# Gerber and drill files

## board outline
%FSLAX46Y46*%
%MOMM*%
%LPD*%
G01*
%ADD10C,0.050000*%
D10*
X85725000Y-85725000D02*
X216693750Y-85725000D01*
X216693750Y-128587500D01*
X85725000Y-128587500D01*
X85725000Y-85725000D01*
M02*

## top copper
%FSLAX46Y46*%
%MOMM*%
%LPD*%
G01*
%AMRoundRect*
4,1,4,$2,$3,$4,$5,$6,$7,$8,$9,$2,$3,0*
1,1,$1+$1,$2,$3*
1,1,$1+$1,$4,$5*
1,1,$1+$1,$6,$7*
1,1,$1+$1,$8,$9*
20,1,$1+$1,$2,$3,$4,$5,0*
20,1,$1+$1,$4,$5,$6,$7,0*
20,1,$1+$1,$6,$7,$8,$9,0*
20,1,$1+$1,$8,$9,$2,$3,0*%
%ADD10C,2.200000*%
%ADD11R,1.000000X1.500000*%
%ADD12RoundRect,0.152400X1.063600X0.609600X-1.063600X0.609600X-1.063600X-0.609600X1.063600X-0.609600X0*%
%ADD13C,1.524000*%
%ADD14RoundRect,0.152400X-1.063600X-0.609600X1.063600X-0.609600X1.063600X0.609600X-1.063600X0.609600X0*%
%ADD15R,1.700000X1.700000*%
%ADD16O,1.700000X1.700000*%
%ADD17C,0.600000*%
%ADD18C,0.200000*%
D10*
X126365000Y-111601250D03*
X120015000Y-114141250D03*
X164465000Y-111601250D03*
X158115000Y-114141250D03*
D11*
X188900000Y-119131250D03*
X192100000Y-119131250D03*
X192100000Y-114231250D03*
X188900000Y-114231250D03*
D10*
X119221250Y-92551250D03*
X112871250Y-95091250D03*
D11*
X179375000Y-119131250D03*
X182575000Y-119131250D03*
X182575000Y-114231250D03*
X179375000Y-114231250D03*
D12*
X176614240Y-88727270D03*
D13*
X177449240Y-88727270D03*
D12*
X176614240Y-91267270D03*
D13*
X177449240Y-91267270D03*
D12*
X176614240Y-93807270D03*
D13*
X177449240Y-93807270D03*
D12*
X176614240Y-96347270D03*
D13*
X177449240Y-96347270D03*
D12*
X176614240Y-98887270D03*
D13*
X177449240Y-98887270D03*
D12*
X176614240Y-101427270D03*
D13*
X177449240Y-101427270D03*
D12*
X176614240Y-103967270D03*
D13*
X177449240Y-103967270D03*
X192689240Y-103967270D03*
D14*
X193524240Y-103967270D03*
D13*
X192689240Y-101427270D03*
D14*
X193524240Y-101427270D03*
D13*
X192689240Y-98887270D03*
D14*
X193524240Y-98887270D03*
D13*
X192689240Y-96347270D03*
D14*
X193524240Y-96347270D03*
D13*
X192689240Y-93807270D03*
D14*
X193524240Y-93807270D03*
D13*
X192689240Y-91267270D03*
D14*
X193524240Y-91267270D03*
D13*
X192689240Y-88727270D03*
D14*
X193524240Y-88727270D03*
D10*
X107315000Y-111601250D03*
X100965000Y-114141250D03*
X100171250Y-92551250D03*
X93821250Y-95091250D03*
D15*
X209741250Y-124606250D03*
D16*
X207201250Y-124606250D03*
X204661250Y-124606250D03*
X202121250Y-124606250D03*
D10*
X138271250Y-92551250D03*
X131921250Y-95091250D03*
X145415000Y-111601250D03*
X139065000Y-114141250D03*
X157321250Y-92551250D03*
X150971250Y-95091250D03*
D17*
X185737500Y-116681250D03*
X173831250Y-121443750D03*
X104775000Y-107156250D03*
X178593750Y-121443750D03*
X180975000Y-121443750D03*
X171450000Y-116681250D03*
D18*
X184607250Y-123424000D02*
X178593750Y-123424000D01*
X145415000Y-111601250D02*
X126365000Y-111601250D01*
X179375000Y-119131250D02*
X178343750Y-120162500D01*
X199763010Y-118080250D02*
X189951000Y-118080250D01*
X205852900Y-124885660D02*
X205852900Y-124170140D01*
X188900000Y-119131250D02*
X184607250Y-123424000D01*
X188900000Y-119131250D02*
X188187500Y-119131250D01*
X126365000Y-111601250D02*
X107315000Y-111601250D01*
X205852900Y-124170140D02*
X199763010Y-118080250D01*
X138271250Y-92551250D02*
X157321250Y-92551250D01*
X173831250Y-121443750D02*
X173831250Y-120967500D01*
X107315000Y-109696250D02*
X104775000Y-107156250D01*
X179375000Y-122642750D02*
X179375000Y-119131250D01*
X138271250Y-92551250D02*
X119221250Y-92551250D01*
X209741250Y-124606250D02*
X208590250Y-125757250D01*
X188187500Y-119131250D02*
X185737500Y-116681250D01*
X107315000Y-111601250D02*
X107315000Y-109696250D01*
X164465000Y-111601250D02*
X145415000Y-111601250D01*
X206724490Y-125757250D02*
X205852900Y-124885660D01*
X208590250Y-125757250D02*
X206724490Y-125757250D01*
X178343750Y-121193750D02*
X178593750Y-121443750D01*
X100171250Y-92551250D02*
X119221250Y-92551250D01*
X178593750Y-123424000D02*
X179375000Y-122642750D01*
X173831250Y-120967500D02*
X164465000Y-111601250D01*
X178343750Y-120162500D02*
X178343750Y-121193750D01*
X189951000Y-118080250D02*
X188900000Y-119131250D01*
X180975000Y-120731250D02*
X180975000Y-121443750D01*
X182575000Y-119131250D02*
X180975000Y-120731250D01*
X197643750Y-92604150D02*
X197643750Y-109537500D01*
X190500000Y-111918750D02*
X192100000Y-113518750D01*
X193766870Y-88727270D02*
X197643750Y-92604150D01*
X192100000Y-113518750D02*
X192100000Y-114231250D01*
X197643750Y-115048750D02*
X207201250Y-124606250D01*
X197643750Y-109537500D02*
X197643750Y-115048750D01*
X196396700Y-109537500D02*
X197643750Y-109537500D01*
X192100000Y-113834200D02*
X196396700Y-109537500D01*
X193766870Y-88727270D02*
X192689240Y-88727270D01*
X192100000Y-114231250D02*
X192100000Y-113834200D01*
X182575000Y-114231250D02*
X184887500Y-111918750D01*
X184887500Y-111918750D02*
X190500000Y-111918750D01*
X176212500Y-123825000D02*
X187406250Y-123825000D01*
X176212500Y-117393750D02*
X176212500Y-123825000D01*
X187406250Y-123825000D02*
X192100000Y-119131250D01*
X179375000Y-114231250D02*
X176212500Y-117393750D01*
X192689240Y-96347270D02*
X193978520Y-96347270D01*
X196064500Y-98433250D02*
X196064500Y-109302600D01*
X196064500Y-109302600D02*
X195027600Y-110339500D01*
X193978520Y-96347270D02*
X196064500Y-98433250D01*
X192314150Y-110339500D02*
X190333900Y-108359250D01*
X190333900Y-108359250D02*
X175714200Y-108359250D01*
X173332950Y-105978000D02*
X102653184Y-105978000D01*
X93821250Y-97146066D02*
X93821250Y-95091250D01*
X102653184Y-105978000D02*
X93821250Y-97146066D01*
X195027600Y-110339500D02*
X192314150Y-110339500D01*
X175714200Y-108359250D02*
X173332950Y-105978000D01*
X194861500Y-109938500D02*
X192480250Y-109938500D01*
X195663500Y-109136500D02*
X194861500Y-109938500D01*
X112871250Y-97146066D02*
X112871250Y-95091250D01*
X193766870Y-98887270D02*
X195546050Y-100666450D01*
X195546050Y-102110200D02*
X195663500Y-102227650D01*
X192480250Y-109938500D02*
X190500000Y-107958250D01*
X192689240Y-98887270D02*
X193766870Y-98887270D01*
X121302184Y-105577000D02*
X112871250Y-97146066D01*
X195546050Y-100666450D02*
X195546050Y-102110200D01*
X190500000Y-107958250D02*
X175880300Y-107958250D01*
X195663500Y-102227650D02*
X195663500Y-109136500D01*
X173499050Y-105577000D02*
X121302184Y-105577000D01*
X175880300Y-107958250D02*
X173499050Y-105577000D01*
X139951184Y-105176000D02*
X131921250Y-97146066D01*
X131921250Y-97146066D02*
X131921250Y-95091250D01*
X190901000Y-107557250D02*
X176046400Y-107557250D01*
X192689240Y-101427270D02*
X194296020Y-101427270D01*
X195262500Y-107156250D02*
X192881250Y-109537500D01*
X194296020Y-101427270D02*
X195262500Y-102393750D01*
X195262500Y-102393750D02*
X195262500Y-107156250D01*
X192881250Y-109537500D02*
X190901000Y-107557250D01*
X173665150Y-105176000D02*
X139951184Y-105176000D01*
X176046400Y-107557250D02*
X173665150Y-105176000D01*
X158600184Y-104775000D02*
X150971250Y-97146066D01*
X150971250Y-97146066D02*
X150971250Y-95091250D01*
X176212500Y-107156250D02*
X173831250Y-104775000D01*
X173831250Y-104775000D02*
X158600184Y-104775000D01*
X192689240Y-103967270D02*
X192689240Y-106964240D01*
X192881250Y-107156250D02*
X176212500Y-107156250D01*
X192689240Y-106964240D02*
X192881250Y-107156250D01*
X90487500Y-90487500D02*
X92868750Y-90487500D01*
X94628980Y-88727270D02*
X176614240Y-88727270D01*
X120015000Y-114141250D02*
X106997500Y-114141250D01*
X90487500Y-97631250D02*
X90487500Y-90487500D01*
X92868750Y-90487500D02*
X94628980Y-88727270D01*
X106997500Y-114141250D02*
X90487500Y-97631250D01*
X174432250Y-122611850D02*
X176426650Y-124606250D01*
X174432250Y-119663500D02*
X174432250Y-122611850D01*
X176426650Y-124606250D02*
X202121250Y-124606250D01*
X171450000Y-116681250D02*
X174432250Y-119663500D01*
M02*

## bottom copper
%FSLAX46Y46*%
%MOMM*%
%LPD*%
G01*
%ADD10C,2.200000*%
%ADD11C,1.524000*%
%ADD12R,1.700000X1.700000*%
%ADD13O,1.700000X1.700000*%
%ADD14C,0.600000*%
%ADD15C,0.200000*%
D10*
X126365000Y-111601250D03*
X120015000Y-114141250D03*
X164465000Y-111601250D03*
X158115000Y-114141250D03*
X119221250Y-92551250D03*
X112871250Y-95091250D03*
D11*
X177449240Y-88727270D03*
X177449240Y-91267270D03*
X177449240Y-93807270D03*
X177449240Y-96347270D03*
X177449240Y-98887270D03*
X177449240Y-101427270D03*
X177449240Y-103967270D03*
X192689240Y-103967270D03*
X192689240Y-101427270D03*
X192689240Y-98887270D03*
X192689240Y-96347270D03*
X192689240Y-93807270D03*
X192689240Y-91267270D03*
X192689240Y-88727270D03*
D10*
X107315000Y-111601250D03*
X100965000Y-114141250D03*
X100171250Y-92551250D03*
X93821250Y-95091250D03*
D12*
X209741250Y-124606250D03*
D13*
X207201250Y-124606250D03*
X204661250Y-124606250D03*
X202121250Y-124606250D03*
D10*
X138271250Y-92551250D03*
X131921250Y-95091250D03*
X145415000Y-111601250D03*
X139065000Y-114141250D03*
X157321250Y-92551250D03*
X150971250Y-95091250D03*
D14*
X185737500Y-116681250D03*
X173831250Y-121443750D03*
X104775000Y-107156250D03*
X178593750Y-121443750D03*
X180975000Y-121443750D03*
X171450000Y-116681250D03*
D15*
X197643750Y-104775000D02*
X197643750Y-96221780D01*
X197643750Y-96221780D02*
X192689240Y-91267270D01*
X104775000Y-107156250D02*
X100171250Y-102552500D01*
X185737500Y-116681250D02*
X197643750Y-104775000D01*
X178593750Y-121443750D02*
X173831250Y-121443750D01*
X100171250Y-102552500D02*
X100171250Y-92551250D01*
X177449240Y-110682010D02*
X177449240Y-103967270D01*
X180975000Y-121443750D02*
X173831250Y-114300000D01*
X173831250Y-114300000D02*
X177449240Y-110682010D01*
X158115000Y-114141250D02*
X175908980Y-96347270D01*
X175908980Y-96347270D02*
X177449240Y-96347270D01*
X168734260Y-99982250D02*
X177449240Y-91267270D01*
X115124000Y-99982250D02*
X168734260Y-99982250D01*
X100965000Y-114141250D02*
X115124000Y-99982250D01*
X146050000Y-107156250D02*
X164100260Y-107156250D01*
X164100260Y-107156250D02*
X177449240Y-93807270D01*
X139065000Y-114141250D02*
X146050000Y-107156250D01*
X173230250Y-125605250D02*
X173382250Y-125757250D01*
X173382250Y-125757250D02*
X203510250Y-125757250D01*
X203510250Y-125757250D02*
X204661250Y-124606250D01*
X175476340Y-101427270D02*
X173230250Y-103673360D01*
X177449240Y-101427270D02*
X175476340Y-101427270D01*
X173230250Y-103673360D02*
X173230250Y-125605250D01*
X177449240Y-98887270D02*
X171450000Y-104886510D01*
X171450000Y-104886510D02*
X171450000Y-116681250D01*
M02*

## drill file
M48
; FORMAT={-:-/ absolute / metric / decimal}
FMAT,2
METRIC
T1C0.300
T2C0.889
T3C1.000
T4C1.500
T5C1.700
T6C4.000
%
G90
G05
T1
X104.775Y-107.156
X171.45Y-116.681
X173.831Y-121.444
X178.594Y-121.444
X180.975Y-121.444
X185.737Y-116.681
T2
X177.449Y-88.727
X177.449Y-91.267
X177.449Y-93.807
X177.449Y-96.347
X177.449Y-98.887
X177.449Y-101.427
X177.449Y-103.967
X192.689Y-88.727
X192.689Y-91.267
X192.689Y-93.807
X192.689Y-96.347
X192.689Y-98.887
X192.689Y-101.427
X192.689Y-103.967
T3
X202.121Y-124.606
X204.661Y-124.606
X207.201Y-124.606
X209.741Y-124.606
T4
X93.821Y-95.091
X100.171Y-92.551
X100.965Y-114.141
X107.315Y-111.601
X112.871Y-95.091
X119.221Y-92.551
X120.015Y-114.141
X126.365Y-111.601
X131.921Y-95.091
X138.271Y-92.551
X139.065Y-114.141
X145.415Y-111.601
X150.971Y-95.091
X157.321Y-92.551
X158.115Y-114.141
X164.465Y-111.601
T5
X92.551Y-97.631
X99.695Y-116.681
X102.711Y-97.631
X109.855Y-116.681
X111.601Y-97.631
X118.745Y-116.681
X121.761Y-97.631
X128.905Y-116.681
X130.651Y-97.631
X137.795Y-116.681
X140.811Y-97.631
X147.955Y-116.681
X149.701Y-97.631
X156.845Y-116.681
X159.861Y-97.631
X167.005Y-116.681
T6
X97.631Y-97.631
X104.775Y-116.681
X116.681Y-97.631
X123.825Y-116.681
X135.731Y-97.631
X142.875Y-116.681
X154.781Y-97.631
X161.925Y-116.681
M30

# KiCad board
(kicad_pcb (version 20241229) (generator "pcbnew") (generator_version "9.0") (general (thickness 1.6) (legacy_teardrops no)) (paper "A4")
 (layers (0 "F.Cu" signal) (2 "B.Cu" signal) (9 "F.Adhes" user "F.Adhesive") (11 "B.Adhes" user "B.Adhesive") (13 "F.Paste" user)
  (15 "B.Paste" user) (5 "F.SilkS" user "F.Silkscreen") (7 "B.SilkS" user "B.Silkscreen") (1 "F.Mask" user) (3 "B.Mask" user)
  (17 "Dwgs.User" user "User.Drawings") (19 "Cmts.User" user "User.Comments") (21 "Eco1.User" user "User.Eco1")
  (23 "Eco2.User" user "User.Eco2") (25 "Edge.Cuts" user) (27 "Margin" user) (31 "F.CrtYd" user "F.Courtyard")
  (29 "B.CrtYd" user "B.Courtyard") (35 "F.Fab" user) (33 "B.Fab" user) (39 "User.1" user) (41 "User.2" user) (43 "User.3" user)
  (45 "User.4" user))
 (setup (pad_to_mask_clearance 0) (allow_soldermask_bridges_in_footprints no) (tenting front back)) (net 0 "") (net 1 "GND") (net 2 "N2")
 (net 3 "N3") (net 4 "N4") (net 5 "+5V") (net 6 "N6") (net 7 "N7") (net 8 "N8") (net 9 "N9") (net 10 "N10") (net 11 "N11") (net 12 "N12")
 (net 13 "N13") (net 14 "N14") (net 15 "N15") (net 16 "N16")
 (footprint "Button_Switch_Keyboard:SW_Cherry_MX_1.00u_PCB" (layer "F.Cu") (at 126.365 111.60125)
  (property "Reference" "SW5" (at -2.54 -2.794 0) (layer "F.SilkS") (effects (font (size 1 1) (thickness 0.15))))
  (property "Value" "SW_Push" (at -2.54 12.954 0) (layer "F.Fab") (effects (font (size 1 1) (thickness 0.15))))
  (pad "" np_thru_hole circle (at -7.62 5.08) (size 1.7 1.7) (drill 1.7) (layers "*.Cu" "*.Mask"))
  (pad "" np_thru_hole circle (at -2.54 5.08) (size 4 4) (drill 4) (layers "*.Cu" "*.Mask"))
  (pad "" np_thru_hole circle (at 2.54 5.08) (size 1.7 1.7) (drill 1.7) (layers "*.Cu" "*.Mask"))
  (pad "1" thru_hole circle (at 0 0) (size 2.2 2.2) (drill 1.5) (layers "*.Cu" "*.Mask") (remove_unused_layers no) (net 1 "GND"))
  (pad "2" thru_hole circle (at -6.35 2.54) (size 2.2 2.2) (drill 1.5) (layers "*.Cu" "*.Mask") (remove_unused_layers no) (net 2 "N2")))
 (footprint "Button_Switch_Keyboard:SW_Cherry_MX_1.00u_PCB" (layer "F.Cu") (at 164.465 111.60125)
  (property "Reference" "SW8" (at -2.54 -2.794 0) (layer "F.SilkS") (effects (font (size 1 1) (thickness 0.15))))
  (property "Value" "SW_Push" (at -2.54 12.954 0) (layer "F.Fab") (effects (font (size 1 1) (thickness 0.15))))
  (pad "" np_thru_hole circle (at -7.62 5.08) (size 1.7 1.7) (drill 1.7) (layers "*.Cu" "*.Mask"))
  (pad "" np_thru_hole circle (at -2.54 5.08) (size 4 4) (drill 4) (layers "*.Cu" "*.Mask"))
  (pad "" np_thru_hole circle (at 2.54 5.08) (size 1.7 1.7) (drill 1.7) (layers "*.Cu" "*.Mask"))
  (pad "1" thru_hole circle (at 0 0) (size 2.2 2.2) (drill 1.5) (layers "*.Cu" "*.Mask") (remove_unused_layers no) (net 1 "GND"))
  (pad "2" thru_hole circle (at -6.35 2.54) (size 2.2 2.2) (drill 1.5) (layers "*.Cu" "*.Mask") (remove_unused_layers no) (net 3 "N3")))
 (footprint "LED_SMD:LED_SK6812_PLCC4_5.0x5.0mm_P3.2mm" (layer "F.Cu") (at 190.5 116.68125 90)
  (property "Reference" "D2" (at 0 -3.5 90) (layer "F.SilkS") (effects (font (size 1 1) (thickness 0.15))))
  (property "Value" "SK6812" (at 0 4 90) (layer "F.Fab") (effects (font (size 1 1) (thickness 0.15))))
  (pad "1" smd rect (at -2.45 -1.6 270) (size 1.5 1) (layers "F.Cu" "F.Mask" "F.Paste") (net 1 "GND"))
  (pad "2" smd rect (at -2.45 1.6 270) (size 1.5 1) (layers "F.Cu" "F.Mask" "F.Paste") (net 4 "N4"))
  (pad "3" smd rect (at 2.45 1.6 270) (size 1.5 1) (layers "F.Cu" "F.Mask" "F.Paste") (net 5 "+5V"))
  (pad "4" smd rect (at 2.45 -1.6 270) (size 1.5 1) (layers "F.Cu" "F.Mask" "F.Paste") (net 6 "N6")))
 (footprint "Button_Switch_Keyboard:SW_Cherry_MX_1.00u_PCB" (layer "F.Cu") (at 119.22125 92.55125)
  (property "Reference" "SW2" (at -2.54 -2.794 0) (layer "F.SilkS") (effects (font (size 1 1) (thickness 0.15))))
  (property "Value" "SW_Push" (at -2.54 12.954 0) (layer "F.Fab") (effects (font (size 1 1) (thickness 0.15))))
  (pad "" np_thru_hole circle (at -7.62 5.08) (size 1.7 1.7) (drill 1.7) (layers "*.Cu" "*.Mask"))
  (pad "" np_thru_hole circle (at -2.54 5.08) (size 4 4) (drill 4) (layers "*.Cu" "*.Mask"))
  (pad "" np_thru_hole circle (at 2.54 5.08) (size 1.7 1.7) (drill 1.7) (layers "*.Cu" "*.Mask"))
  (pad "1" thru_hole circle (at 0 0) (size 2.2 2.2) (drill 1.5) (layers "*.Cu" "*.Mask") (remove_unused_layers no) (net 1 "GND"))
  (pad "2" thru_hole circle (at -6.35 2.54) (size 2.2 2.2) (drill 1.5) (layers "*.Cu" "*.Mask") (remove_unused_layers no) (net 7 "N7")))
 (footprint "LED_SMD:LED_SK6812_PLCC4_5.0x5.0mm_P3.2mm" (layer "F.Cu") (at 180.975 116.68125 90)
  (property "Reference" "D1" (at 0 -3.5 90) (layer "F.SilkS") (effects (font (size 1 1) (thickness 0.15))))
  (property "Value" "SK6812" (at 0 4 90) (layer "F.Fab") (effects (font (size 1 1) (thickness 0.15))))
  (pad "1" smd rect (at -2.45 -1.6 270) (size 1.5 1) (layers "F.Cu" "F.Mask" "F.Paste") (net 1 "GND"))
  (pad "2" smd rect (at -2.45 1.6 270) (size 1.5 1) (layers "F.Cu" "F.Mask" "F.Paste") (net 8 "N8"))
  (pad "3" smd rect (at 2.45 1.6 270) (size 1.5 1) (layers "F.Cu" "F.Mask" "F.Paste") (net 5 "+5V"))
  (pad "4" smd rect (at 2.45 -1.6 270) (size 1.5 1) (layers "F.Cu" "F.Mask" "F.Paste") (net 4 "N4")))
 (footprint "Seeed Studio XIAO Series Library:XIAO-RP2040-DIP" (layer "F.Cu") (at 185.06924 96.34727)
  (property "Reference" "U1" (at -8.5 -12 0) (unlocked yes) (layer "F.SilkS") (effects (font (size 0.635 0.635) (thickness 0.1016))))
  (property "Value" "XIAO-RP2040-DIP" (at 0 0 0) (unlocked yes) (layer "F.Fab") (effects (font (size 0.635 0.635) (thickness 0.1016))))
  (pad "1" smd roundrect (at -8.455 -7.62 180) (size 2.432 1.524) (layers "F.Cu" "F.Mask") (roundrect_rratio 0.1) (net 2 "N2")
   (thermal_bridge_angle 45))
  (pad "1" thru_hole circle (at -7.62 -7.62 180) (size 1.524 1.524) (drill 0.889) (layers "*.Cu" "*.Mask") (remove_unused_layers no)
   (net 2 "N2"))
  (pad "2" smd roundrect (at -8.455 -5.08 180) (size 2.432 1.524) (layers "F.Cu" "F.Mask") (roundrect_rratio 0.1) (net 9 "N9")
   (thermal_bridge_angle 45))
  (pad "2" thru_hole circle (at -7.62 -5.08 180) (size 1.524 1.524) (drill 0.889) (layers "*.Cu" "*.Mask") (remove_unused_layers no)
   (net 9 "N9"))
  (pad "3" smd roundrect (at -8.455 -2.54 180) (size 2.432 1.524) (layers "F.Cu" "F.Mask") (roundrect_rratio 0.1) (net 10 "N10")
   (thermal_bridge_angle 45))
  (pad "3" thru_hole circle (at -7.62 -2.54 180) (size 1.524 1.524) (drill 0.889) (layers "*.Cu" "*.Mask") (remove_unused_layers no)
   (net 10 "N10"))
  (pad "4" smd roundrect (at -8.455 0 180) (size 2.432 1.524) (layers "F.Cu" "F.Mask") (roundrect_rratio 0.1) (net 3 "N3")
   (thermal_bridge_angle 45))
  (pad "4" thru_hole circle (at -7.62 0 180) (size 1.524 1.524) (drill 0.889) (layers "*.Cu" "*.Mask") (remove_unused_layers no)
   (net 3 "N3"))
  (pad "5" smd roundrect (at -8.455 2.54 180) (size 2.432 1.524) (layers "F.Cu" "F.Mask") (roundrect_rratio 0.1) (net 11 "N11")
   (thermal_bridge_angle 45))
  (pad "5" thru_hole circle (at -7.62 2.54 180) (size 1.524 1.524) (drill 0.889) (layers "*.Cu" "*.Mask") (remove_unused_layers no)
   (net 11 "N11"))
  (pad "6" smd roundrect (at -8.455 5.08 180) (size 2.432 1.524) (layers "F.Cu" "F.Mask") (roundrect_rratio 0.1) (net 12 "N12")
   (thermal_bridge_angle 45))
  (pad "6" thru_hole circle (at -7.62 5.08 180) (size 1.524 1.524) (drill 0.889) (layers "*.Cu" "*.Mask") (remove_unused_layers no)
   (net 12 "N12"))
  (pad "7" smd roundrect (at -8.455 7.62 180) (size 2.432 1.524) (layers "F.Cu" "F.Mask") (roundrect_rratio 0.1) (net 8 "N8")
   (thermal_bridge_angle 45))
  (pad "7" thru_hole circle (at -7.62 7.62 180) (size 1.524 1.524) (drill 0.889) (layers "*.Cu" "*.Mask") (remove_unused_layers no)
   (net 8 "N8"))
  (pad "8" thru_hole circle (at 7.62 7.62) (size 1.524 1.524) (drill 0.889) (layers "*.Cu" "*.Mask") (remove_unused_layers no)
   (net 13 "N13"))
  (pad "8" smd roundrect (at 8.455 7.62) (size 2.432 1.524) (layers "F.Cu" "F.Mask") (roundrect_rratio 0.1) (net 13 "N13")
   (thermal_bridge_angle 45))
  (pad "9" thru_hole circle (at 7.62 5.08) (size 1.524 1.524) (drill 0.889) (layers "*.Cu" "*.Mask") (remove_unused_layers no)
   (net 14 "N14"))
  (pad "9" smd roundrect (at 8.455 5.08) (size 2.432 1.524) (layers "F.Cu" "F.Mask") (roundrect_rratio 0.1) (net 14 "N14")
   (thermal_bridge_angle 45))
  (pad "10" thru_hole circle (at 7.62 2.54) (size 1.524 1.524) (drill 0.889) (layers "*.Cu" "*.Mask") (remove_unused_layers no) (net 7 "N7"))
  (pad "10" smd roundrect (at 8.455 2.54) (size 2.432 1.524) (layers "F.Cu" "F.Mask") (roundrect_rratio 0.1) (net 7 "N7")
   (thermal_bridge_angle 45))
  (pad "11" thru_hole circle (at 7.62 0) (size 1.524 1.524) (drill 0.889) (layers "*.Cu" "*.Mask") (remove_unused_layers no) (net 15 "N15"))
  (pad "11" smd roundrect (at 8.455 0) (size 2.432 1.524) (layers "F.Cu" "F.Mask") (roundrect_rratio 0.1) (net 15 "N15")
   (thermal_bridge_angle 45))
  (pad "12" thru_hole circle (at 7.62 -2.54) (size 1.524 1.524) (drill 0.889) (layers "*.Cu" "*.Mask") (remove_unused_layers no)
   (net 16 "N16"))
  (pad "12" smd roundrect (at 8.455 -2.54) (size 2.432 1.524) (layers "F.Cu" "F.Mask") (roundrect_rratio 0.1) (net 16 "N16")
   (thermal_bridge_angle 45))
  (pad "13" thru_hole circle (at 7.62 -5.08) (size 1.524 1.524) (drill 0.889) (layers "*.Cu" "*.Mask") (remove_unused_layers no)
   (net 1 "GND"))
  (pad "13" smd roundrect (at 8.455 -5.08) (size 2.432 1.524) (layers "F.Cu" "F.Mask") (roundrect_rratio 0.1) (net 1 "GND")
   (thermal_bridge_angle 45))
  (pad "14" thru_hole circle (at 7.62 -7.62) (size 1.524 1.524) (drill 0.889) (layers "*.Cu" "*.Mask") (remove_unused_layers no)
   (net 5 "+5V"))
  (pad "14" smd roundrect (at 8.455 -7.62) (size 2.432 1.524) (layers "F.Cu" "F.Mask") (roundrect_rratio 0.1) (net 5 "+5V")
   (thermal_bridge_angle 45)))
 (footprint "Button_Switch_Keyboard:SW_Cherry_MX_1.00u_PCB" (layer "F.Cu") (at 107.315 111.60125)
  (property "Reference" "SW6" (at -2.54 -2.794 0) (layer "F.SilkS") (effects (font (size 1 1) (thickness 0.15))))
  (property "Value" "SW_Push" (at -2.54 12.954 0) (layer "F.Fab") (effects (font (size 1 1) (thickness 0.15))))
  (pad "" np_thru_hole circle (at -7.62 5.08) (size 1.7 1.7) (drill 1.7) (layers "*.Cu" "*.Mask"))
  (pad "" np_thru_hole circle (at -2.54 5.08) (size 4 4) (drill 4) (layers "*.Cu" "*.Mask"))
  (pad "" np_thru_hole circle (at 2.54 5.08) (size 1.7 1.7) (drill 1.7) (layers "*.Cu" "*.Mask"))
  (pad "1" thru_hole circle (at 0 0) (size 2.2 2.2) (drill 1.5) (layers "*.Cu" "*.Mask") (remove_unused_layers no) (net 1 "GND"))
  (pad "2" thru_hole circle (at -6.35 2.54) (size 2.2 2.2) (drill 1.5) (layers "*.Cu" "*.Mask") (remove_unused_layers no) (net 9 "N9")))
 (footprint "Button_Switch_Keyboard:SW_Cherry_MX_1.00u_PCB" (layer "F.Cu") (at 100.17125 92.55125)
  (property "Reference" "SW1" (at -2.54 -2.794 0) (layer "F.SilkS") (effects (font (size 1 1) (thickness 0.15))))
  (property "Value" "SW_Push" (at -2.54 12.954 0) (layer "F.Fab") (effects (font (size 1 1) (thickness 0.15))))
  (pad "" np_thru_hole circle (at -7.62 5.08) (size 1.7 1.7) (drill 1.7) (layers "*.Cu" "*.Mask"))
  (pad "" np_thru_hole circle (at -2.54 5.08) (size 4 4) (drill 4) (layers "*.Cu" "*.Mask"))
  (pad "" np_thru_hole circle (at 2.54 5.08) (size 1.7 1.7) (drill 1.7) (layers "*.Cu" "*.Mask"))
  (pad "1" thru_hole circle (at 0 0) (size 2.2 2.2) (drill 1.5) (layers "*.Cu" "*.Mask") (remove_unused_layers no) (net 1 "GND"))
  (pad "2" thru_hole circle (at -6.35 2.54) (size 2.2 2.2) (drill 1.5) (layers "*.Cu" "*.Mask") (remove_unused_layers no) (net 15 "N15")))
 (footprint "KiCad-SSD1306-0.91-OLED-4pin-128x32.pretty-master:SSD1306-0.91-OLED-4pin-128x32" (layer "F.Cu") (at 211.93125 88.10625 -90)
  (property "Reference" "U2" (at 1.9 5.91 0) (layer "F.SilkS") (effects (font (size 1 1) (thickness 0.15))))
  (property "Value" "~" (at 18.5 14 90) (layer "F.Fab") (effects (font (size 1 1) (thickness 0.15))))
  (pad "1" thru_hole rect (at 36.5 2.19 270) (size 1.7 1.7) (drill 1) (layers "*.Cu" "*.Mask") (remove_unused_layers no) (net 1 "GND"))
  (pad "2" thru_hole oval (at 36.5 4.73 270) (size 1.7 1.7) (drill 1) (layers "*.Cu" "*.Mask") (remove_unused_layers no) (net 5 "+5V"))
  (pad "3" thru_hole oval (at 36.5 7.27 270) (size 1.7 1.7) (drill 1) (layers "*.Cu" "*.Mask") (remove_unused_layers no) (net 12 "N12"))
  (pad "4" thru_hole oval (at 36.5 9.81 270) (size 1.7 1.7) (drill 1) (layers "*.Cu" "*.Mask") (remove_unused_layers no) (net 11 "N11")))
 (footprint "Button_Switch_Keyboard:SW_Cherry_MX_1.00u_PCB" (layer "F.Cu") (at 138.27125 92.55125)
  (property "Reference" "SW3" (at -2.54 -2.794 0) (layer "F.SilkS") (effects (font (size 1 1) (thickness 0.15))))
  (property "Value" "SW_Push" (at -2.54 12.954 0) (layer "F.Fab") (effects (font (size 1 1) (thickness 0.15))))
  (pad "" np_thru_hole circle (at -7.62 5.08) (size 1.7 1.7) (drill 1.7) (layers "*.Cu" "*.Mask"))
  (pad "" np_thru_hole circle (at -2.54 5.08) (size 4 4) (drill 4) (layers "*.Cu" "*.Mask"))
  (pad "" np_thru_hole circle (at 2.54 5.08) (size 1.7 1.7) (drill 1.7) (layers "*.Cu" "*.Mask"))
  (pad "1" thru_hole circle (at 0 0) (size 2.2 2.2) (drill 1.5) (layers "*.Cu" "*.Mask") (remove_unused_layers no) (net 1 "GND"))
  (pad "2" thru_hole circle (at -6.35 2.54) (size 2.2 2.2) (drill 1.5) (layers "*.Cu" "*.Mask") (remove_unused_layers no) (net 14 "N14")))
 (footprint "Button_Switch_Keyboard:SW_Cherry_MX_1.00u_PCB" (layer "F.Cu") (at 145.415 111.60125)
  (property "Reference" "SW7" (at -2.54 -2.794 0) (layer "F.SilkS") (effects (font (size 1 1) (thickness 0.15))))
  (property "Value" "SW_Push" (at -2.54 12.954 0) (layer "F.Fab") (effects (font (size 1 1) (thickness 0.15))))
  (pad "" np_thru_hole circle (at -7.62 5.08) (size 1.7 1.7) (drill 1.7) (layers "*.Cu" "*.Mask"))
  (pad "" np_thru_hole circle (at -2.54 5.08) (size 4 4) (drill 4) (layers "*.Cu" "*.Mask"))
  (pad "" np_thru_hole circle (at 2.54 5.08) (size 1.7 1.7) (drill 1.7) (layers "*.Cu" "*.Mask"))
  (pad "1" thru_hole circle (at 0 0) (size 2.2 2.2) (drill 1.5) (layers "*.Cu" "*.Mask") (remove_unused_layers no) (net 1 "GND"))
  (pad "2" thru_hole circle (at -6.35 2.54) (size 2.2 2.2) (drill 1.5) (layers "*.Cu" "*.Mask") (remove_unused_layers no) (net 10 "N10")))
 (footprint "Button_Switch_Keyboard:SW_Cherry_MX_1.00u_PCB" (layer "F.Cu") (at 157.32125 92.55125)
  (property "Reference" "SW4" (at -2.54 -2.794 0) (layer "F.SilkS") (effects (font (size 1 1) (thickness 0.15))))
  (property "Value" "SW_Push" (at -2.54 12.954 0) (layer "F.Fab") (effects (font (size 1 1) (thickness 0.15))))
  (pad "" np_thru_hole circle (at -7.62 5.08) (size 1.7 1.7) (drill 1.7) (layers "*.Cu" "*.Mask"))
  (pad "" np_thru_hole circle (at -2.54 5.08) (size 4 4) (drill 4) (layers "*.Cu" "*.Mask"))
  (pad "" np_thru_hole circle (at 2.54 5.08) (size 1.7 1.7) (drill 1.7) (layers "*.Cu" "*.Mask"))
  (pad "1" thru_hole circle (at 0 0) (size 2.2 2.2) (drill 1.5) (layers "*.Cu" "*.Mask") (remove_unused_layers no) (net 1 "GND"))
  (pad "2" thru_hole circle (at -6.35 2.54) (size 2.2 2.2) (drill 1.5) (layers "*.Cu" "*.Mask") (remove_unused_layers no) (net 13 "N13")))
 (gr_rect (start 85.725 85.725) (end 216.69375 128.5875) (stroke (width 0.05) (type default)) (fill no) (layer "Edge.Cuts"))
 (segment (start 184.60725 123.424) (end 178.59375 123.424) (width 0.2) (layer "F.Cu") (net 1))
 (segment (start 145.415 111.60125) (end 126.365 111.60125) (width 0.2) (layer "F.Cu") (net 1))
 (segment (start 179.375 119.13125) (end 178.34375 120.1625) (width 0.2) (layer "F.Cu") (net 1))
 (segment (start 199.76301 118.08025) (end 189.951 118.08025) (width 0.2) (layer "F.Cu") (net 1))
 (segment (start 205.8529 124.88566) (end 205.8529 124.17014) (width 0.2) (layer "F.Cu") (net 1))
 (segment (start 188.9 119.13125) (end 184.60725 123.424) (width 0.2) (layer "F.Cu") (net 1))
 (segment (start 188.9 119.13125) (end 188.1875 119.13125) (width 0.2) (layer "F.Cu") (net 1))
 (segment (start 126.365 111.60125) (end 107.315 111.60125) (width 0.2) (layer "F.Cu") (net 1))
 (segment (start 205.8529 124.17014) (end 199.76301 118.08025) (width 0.2) (layer "F.Cu") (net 1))
 (segment (start 138.27125 92.55125) (end 157.32125 92.55125) (width 0.2) (layer "F.Cu") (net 1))
 (segment (start 173.83125 121.44375) (end 173.83125 120.9675) (width 0.2) (layer "F.Cu") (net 1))
 (segment (start 107.315 109.69625) (end 104.775 107.15625) (width 0.2) (layer "F.Cu") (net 1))
 (segment (start 179.375 122.64275) (end 179.375 119.13125) (width 0.2) (layer "F.Cu") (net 1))
 (segment (start 138.27125 92.55125) (end 119.22125 92.55125) (width 0.2) (layer "F.Cu") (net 1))
 (segment (start 209.74125 124.60625) (end 208.59025 125.75725) (width 0.2) (layer "F.Cu") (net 1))
 (segment (start 188.1875 119.13125) (end 185.7375 116.68125) (width 0.2) (layer "F.Cu") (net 1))
 (segment (start 107.315 111.60125) (end 107.315 109.69625) (width 0.2) (layer "F.Cu") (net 1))
 (segment (start 164.465 111.60125) (end 145.415 111.60125) (width 0.2) (layer "F.Cu") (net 1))
 (segment (start 206.72449 125.75725) (end 205.8529 124.88566) (width 0.2) (layer "F.Cu") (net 1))
 (segment (start 208.59025 125.75725) (end 206.72449 125.75725) (width 0.2) (layer "F.Cu") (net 1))
 (segment (start 178.34375 121.19375) (end 178.59375 121.44375) (width 0.2) (layer "F.Cu") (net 1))
 (segment (start 100.17125 92.55125) (end 119.22125 92.55125) (width 0.2) (layer "F.Cu") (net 1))
 (segment (start 178.59375 123.424) (end 179.375 122.64275) (width 0.2) (layer "F.Cu") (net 1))
 (segment (start 173.83125 120.9675) (end 164.465 111.60125) (width 0.2) (layer "F.Cu") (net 1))
 (segment (start 178.34375 120.1625) (end 178.34375 121.19375) (width 0.2) (layer "F.Cu") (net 1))
 (segment (start 189.951 118.08025) (end 188.9 119.13125) (width 0.2) (layer "F.Cu") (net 1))
 (via (at 185.7375 116.68125) (size 0.6) (drill 0.3) (layers "F.Cu" "B.Cu") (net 1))
 (via (at 173.83125 121.44375) (size 0.6) (drill 0.3) (layers "F.Cu" "B.Cu") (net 1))
 (via (at 104.775 107.15625) (size 0.6) (drill 0.3) (layers "F.Cu" "B.Cu") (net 1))
 (via (at 178.59375 121.44375) (size 0.6) (drill 0.3) (layers "F.Cu" "B.Cu") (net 1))
 (segment (start 197.64375 104.775) (end 197.64375 96.22178) (width 0.2) (layer "B.Cu") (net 1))
 (segment (start 197.64375 96.22178) (end 192.68924 91.26727) (width 0.2) (layer "B.Cu") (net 1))
 (segment (start 104.775 107.15625) (end 100.17125 102.5525) (width 0.2) (layer "B.Cu") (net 1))
 (segment (start 185.7375 116.68125) (end 197.64375 104.775) (width 0.2) (layer "B.Cu") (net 1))
 (segment (start 178.59375 121.44375) (end 173.83125 121.44375) (width 0.2) (layer "B.Cu") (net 1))
 (segment (start 100.17125 102.5525) (end 100.17125 92.55125) (width 0.2) (layer "B.Cu") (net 1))
 (segment (start 180.975 120.73125) (end 180.975 121.44375) (width 0.2) (layer "F.Cu") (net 8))
 (segment (start 182.575 119.13125) (end 180.975 120.73125) (width 0.2) (layer "F.Cu") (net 8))
 (via (at 180.975 121.44375) (size 0.6) (drill 0.3) (layers "F.Cu" "B.Cu") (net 8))
 (segment (start 177.44924 110.68201) (end 177.44924 103.96727) (width 0.2) (layer "B.Cu") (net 8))
 (segment (start 180.975 121.44375) (end 173.83125 114.3) (width 0.2) (layer "B.Cu") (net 8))
 (segment (start 173.83125 114.3) (end 177.44924 110.68201) (width 0.2) (layer "B.Cu") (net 8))
 (segment (start 197.64375 92.60415) (end 197.64375 109.5375) (width 0.2) (layer "F.Cu") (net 5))
 (segment (start 190.5 111.91875) (end 192.1 113.51875) (width 0.2) (layer "F.Cu") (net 5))
 (segment (start 193.76687 88.72727) (end 197.64375 92.60415) (width 0.2) (layer "F.Cu") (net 5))
 (segment (start 192.1 113.51875) (end 192.1 114.23125) (width 0.2) (layer "F.Cu") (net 5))
 (segment (start 197.64375 115.04875) (end 207.20125 124.60625) (width 0.2) (layer "F.Cu") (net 5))
 (segment (start 197.64375 109.5375) (end 197.64375 115.04875) (width 0.2) (layer "F.Cu") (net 5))
 (segment (start 196.3967 109.5375) (end 197.64375 109.5375) (width 0.2) (layer "F.Cu") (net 5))
 (segment (start 192.1 113.8342) (end 196.3967 109.5375) (width 0.2) (layer "F.Cu") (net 5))
 (segment (start 193.76687 88.72727) (end 192.68924 88.72727) (width 0.2) (layer "F.Cu") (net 5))
 (segment (start 192.1 114.23125) (end 192.1 113.8342) (width 0.2) (layer "F.Cu") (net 5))
 (segment (start 182.575 114.23125) (end 184.8875 111.91875) (width 0.2) (layer "F.Cu") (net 5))
 (segment (start 184.8875 111.91875) (end 190.5 111.91875) (width 0.2) (layer "F.Cu") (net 5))
 (segment (start 176.2125 123.825) (end 187.40625 123.825) (width 0.2) (layer "F.Cu") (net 4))
 (segment (start 176.2125 117.39375) (end 176.2125 123.825) (width 0.2) (layer "F.Cu") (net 4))
 (segment (start 187.40625 123.825) (end 192.1 119.13125) (width 0.2) (layer "F.Cu") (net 4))
 (segment (start 179.375 114.23125) (end 176.2125 117.39375) (width 0.2) (layer "F.Cu") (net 4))
 (segment (start 158.115 114.14125) (end 175.90898 96.34727) (width 0.2) (layer "B.Cu") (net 3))
 (segment (start 175.90898 96.34727) (end 177.44924 96.34727) (width 0.2) (layer "B.Cu") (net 3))
 (segment (start 192.68924 96.34727) (end 193.97852 96.34727) (width 0.2) (layer "F.Cu") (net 15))
 (segment (start 196.0645 98.43325) (end 196.0645 109.3026) (width 0.2) (layer "F.Cu") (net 15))
 (segment (start 196.0645 109.3026) (end 195.0276 110.3395) (width 0.2) (layer "F.Cu") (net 15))
 (segment (start 193.97852 96.34727) (end 196.0645 98.43325) (width 0.2) (layer "F.Cu") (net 15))
 (segment (start 192.31415 110.3395) (end 190.3339 108.35925) (width 0.2) (layer "F.Cu") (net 15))
 (segment (start 190.3339 108.35925) (end 175.7142 108.35925) (width 0.2) (layer "F.Cu") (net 15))
 (segment (start 173.33295 105.978) (end 102.653184 105.978) (width 0.2) (layer "F.Cu") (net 15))
 (segment (start 93.82125 97.146066) (end 93.82125 95.09125) (width 0.2) (layer "F.Cu") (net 15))
 (segment (start 102.653184 105.978) (end 93.82125 97.146066) (width 0.2) (layer "F.Cu") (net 15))
 (segment (start 195.0276 110.3395) (end 192.31415 110.3395) (width 0.2) (layer "F.Cu") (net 15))
 (segment (start 175.7142 108.35925) (end 173.33295 105.978) (width 0.2) (layer "F.Cu") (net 15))
 (segment (start 194.8615 109.9385) (end 192.48025 109.9385) (width 0.2) (layer "F.Cu") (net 7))
 (segment (start 195.6635 109.1365) (end 194.8615 109.9385) (width 0.2) (layer "F.Cu") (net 7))
 (segment (start 112.87125 97.146066) (end 112.87125 95.09125) (width 0.2) (layer "F.Cu") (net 7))
 (segment (start 193.76687 98.88727) (end 195.54605 100.66645) (width 0.2) (layer "F.Cu") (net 7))
 (segment (start 195.54605 102.1102) (end 195.6635 102.22765) (width 0.2) (layer "F.Cu") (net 7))
 (segment (start 192.48025 109.9385) (end 190.5 107.95825) (width 0.2) (layer "F.Cu") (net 7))
 (segment (start 192.68924 98.88727) (end 193.76687 98.88727) (width 0.2) (layer "F.Cu") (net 7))
 (segment (start 121.302184 105.577) (end 112.87125 97.146066) (width 0.2) (layer "F.Cu") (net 7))
 (segment (start 195.54605 100.66645) (end 195.54605 102.1102) (width 0.2) (layer "F.Cu") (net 7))
 (segment (start 190.5 107.95825) (end 175.8803 107.95825) (width 0.2) (layer "F.Cu") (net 7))
 (segment (start 195.6635 102.22765) (end 195.6635 109.1365) (width 0.2) (layer "F.Cu") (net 7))
 (segment (start 173.49905 105.577) (end 121.302184 105.577) (width 0.2) (layer "F.Cu") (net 7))
 (segment (start 175.8803 107.95825) (end 173.49905 105.577) (width 0.2) (layer "F.Cu") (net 7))
 (segment (start 139.951184 105.176) (end 131.92125 97.146066) (width 0.2) (layer "F.Cu") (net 14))
 (segment (start 131.92125 97.146066) (end 131.92125 95.09125) (width 0.2) (layer "F.Cu") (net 14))
 (segment (start 190.901 107.55725) (end 176.0464 107.55725) (width 0.2) (layer "F.Cu") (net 14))
 (segment (start 192.68924 101.42727) (end 194.29602 101.42727) (width 0.2) (layer "F.Cu") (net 14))
 (segment (start 195.2625 107.15625) (end 192.88125 109.5375) (width 0.2) (layer "F.Cu") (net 14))
 (segment (start 194.29602 101.42727) (end 195.2625 102.39375) (width 0.2) (layer "F.Cu") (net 14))
 (segment (start 195.2625 102.39375) (end 195.2625 107.15625) (width 0.2) (layer "F.Cu") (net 14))
 (segment (start 192.88125 109.5375) (end 190.901 107.55725) (width 0.2) (layer "F.Cu") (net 14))
 (segment (start 173.66515 105.176) (end 139.951184 105.176) (width 0.2) (layer "F.Cu") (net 14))
 (segment (start 176.0464 107.55725) (end 173.66515 105.176) (width 0.2) (layer "F.Cu") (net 14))
 (segment (start 158.600184 104.775) (end 150.97125 97.146066) (width 0.2) (layer "F.Cu") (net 13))
 (segment (start 150.97125 97.146066) (end 150.97125 95.09125) (width 0.2) (layer "F.Cu") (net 13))
 (segment (start 176.2125 107.15625) (end 173.83125 104.775) (width 0.2) (layer "F.Cu") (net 13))
 (segment (start 173.83125 104.775) (end 158.600184 104.775) (width 0.2) (layer "F.Cu") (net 13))
 (segment (start 192.68924 103.96727) (end 192.68924 106.96424) (width 0.2) (layer "F.Cu") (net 13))
 (segment (start 192.88125 107.15625) (end 176.2125 107.15625) (width 0.2) (layer "F.Cu") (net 13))
 (segment (start 192.68924 106.96424) (end 192.88125 107.15625) (width 0.2) (layer "F.Cu") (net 13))
 (segment (start 90.4875 90.4875) (end 92.86875 90.4875) (width 0.2) (layer "F.Cu") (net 2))
 (segment (start 94.62898 88.72727) (end 176.61424 88.72727) (width 0.2) (layer "F.Cu") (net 2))
 (segment (start 120.015 114.14125) (end 106.9975 114.14125) (width 0.2) (layer "F.Cu") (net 2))
 (segment (start 90.4875 97.63125) (end 90.4875 90.4875) (width 0.2) (layer "F.Cu") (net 2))
 (segment (start 92.86875 90.4875) (end 94.62898 88.72727) (width 0.2) (layer "F.Cu") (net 2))
 (segment (start 106.9975 114.14125) (end 90.4875 97.63125) (width 0.2) (layer "F.Cu") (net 2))
 (segment (start 168.73426 99.98225) (end 177.44924 91.26727) (width 0.2) (layer "B.Cu") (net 9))
 (segment (start 115.124 99.98225) (end 168.73426 99.98225) (width 0.2) (layer "B.Cu") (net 9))
 (segment (start 100.965 114.14125) (end 115.124 99.98225) (width 0.2) (layer "B.Cu") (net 9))
 (segment (start 146.05 107.15625) (end 164.10026 107.15625) (width 0.2) (layer "B.Cu") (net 10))
 (segment (start 164.10026 107.15625) (end 177.44924 93.80727) (width 0.2) (layer "B.Cu") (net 10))
 (segment (start 139.065 114.14125) (end 146.05 107.15625) (width 0.2) (layer "B.Cu") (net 10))
 (segment (start 173.23025 125.60525) (end 173.38225 125.75725) (width 0.2) (layer "B.Cu") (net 12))
 (segment (start 173.38225 125.75725) (end 203.51025 125.75725) (width 0.2) (layer "B.Cu") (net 12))
 (segment (start 203.51025 125.75725) (end 204.66125 124.60625) (width 0.2) (layer "B.Cu") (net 12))
 (segment (start 175.47634 101.42727) (end 173.23025 103.67336) (width 0.2) (layer "B.Cu") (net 12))
 (segment (start 177.44924 101.42727) (end 175.47634 101.42727) (width 0.2) (layer "B.Cu") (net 12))
 (segment (start 173.23025 103.67336) (end 173.23025 125.60525) (width 0.2) (layer "B.Cu") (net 12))
 (segment (start 174.43225 122.61185) (end 176.42665 124.60625) (width 0.2) (layer "F.Cu") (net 11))
 (segment (start 174.43225 119.6635) (end 174.43225 122.61185) (width 0.2) (layer "F.Cu") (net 11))
 (segment (start 176.42665 124.60625) (end 202.12125 124.60625) (width 0.2) (layer "F.Cu") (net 11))
 (segment (start 171.45 116.68125) (end 174.43225 119.6635) (width 0.2) (layer "F.Cu") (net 11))
 (via (at 171.45 116.68125) (size 0.6) (drill 0.3) (layers "F.Cu" "B.Cu") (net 11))
 (segment (start 177.44924 98.88727) (end 171.45 104.88651) (width 0.2) (layer "B.Cu") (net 11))
 (segment (start 171.45 104.88651) (end 171.45 116.68125) (width 0.2) (layer "B.Cu") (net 11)))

